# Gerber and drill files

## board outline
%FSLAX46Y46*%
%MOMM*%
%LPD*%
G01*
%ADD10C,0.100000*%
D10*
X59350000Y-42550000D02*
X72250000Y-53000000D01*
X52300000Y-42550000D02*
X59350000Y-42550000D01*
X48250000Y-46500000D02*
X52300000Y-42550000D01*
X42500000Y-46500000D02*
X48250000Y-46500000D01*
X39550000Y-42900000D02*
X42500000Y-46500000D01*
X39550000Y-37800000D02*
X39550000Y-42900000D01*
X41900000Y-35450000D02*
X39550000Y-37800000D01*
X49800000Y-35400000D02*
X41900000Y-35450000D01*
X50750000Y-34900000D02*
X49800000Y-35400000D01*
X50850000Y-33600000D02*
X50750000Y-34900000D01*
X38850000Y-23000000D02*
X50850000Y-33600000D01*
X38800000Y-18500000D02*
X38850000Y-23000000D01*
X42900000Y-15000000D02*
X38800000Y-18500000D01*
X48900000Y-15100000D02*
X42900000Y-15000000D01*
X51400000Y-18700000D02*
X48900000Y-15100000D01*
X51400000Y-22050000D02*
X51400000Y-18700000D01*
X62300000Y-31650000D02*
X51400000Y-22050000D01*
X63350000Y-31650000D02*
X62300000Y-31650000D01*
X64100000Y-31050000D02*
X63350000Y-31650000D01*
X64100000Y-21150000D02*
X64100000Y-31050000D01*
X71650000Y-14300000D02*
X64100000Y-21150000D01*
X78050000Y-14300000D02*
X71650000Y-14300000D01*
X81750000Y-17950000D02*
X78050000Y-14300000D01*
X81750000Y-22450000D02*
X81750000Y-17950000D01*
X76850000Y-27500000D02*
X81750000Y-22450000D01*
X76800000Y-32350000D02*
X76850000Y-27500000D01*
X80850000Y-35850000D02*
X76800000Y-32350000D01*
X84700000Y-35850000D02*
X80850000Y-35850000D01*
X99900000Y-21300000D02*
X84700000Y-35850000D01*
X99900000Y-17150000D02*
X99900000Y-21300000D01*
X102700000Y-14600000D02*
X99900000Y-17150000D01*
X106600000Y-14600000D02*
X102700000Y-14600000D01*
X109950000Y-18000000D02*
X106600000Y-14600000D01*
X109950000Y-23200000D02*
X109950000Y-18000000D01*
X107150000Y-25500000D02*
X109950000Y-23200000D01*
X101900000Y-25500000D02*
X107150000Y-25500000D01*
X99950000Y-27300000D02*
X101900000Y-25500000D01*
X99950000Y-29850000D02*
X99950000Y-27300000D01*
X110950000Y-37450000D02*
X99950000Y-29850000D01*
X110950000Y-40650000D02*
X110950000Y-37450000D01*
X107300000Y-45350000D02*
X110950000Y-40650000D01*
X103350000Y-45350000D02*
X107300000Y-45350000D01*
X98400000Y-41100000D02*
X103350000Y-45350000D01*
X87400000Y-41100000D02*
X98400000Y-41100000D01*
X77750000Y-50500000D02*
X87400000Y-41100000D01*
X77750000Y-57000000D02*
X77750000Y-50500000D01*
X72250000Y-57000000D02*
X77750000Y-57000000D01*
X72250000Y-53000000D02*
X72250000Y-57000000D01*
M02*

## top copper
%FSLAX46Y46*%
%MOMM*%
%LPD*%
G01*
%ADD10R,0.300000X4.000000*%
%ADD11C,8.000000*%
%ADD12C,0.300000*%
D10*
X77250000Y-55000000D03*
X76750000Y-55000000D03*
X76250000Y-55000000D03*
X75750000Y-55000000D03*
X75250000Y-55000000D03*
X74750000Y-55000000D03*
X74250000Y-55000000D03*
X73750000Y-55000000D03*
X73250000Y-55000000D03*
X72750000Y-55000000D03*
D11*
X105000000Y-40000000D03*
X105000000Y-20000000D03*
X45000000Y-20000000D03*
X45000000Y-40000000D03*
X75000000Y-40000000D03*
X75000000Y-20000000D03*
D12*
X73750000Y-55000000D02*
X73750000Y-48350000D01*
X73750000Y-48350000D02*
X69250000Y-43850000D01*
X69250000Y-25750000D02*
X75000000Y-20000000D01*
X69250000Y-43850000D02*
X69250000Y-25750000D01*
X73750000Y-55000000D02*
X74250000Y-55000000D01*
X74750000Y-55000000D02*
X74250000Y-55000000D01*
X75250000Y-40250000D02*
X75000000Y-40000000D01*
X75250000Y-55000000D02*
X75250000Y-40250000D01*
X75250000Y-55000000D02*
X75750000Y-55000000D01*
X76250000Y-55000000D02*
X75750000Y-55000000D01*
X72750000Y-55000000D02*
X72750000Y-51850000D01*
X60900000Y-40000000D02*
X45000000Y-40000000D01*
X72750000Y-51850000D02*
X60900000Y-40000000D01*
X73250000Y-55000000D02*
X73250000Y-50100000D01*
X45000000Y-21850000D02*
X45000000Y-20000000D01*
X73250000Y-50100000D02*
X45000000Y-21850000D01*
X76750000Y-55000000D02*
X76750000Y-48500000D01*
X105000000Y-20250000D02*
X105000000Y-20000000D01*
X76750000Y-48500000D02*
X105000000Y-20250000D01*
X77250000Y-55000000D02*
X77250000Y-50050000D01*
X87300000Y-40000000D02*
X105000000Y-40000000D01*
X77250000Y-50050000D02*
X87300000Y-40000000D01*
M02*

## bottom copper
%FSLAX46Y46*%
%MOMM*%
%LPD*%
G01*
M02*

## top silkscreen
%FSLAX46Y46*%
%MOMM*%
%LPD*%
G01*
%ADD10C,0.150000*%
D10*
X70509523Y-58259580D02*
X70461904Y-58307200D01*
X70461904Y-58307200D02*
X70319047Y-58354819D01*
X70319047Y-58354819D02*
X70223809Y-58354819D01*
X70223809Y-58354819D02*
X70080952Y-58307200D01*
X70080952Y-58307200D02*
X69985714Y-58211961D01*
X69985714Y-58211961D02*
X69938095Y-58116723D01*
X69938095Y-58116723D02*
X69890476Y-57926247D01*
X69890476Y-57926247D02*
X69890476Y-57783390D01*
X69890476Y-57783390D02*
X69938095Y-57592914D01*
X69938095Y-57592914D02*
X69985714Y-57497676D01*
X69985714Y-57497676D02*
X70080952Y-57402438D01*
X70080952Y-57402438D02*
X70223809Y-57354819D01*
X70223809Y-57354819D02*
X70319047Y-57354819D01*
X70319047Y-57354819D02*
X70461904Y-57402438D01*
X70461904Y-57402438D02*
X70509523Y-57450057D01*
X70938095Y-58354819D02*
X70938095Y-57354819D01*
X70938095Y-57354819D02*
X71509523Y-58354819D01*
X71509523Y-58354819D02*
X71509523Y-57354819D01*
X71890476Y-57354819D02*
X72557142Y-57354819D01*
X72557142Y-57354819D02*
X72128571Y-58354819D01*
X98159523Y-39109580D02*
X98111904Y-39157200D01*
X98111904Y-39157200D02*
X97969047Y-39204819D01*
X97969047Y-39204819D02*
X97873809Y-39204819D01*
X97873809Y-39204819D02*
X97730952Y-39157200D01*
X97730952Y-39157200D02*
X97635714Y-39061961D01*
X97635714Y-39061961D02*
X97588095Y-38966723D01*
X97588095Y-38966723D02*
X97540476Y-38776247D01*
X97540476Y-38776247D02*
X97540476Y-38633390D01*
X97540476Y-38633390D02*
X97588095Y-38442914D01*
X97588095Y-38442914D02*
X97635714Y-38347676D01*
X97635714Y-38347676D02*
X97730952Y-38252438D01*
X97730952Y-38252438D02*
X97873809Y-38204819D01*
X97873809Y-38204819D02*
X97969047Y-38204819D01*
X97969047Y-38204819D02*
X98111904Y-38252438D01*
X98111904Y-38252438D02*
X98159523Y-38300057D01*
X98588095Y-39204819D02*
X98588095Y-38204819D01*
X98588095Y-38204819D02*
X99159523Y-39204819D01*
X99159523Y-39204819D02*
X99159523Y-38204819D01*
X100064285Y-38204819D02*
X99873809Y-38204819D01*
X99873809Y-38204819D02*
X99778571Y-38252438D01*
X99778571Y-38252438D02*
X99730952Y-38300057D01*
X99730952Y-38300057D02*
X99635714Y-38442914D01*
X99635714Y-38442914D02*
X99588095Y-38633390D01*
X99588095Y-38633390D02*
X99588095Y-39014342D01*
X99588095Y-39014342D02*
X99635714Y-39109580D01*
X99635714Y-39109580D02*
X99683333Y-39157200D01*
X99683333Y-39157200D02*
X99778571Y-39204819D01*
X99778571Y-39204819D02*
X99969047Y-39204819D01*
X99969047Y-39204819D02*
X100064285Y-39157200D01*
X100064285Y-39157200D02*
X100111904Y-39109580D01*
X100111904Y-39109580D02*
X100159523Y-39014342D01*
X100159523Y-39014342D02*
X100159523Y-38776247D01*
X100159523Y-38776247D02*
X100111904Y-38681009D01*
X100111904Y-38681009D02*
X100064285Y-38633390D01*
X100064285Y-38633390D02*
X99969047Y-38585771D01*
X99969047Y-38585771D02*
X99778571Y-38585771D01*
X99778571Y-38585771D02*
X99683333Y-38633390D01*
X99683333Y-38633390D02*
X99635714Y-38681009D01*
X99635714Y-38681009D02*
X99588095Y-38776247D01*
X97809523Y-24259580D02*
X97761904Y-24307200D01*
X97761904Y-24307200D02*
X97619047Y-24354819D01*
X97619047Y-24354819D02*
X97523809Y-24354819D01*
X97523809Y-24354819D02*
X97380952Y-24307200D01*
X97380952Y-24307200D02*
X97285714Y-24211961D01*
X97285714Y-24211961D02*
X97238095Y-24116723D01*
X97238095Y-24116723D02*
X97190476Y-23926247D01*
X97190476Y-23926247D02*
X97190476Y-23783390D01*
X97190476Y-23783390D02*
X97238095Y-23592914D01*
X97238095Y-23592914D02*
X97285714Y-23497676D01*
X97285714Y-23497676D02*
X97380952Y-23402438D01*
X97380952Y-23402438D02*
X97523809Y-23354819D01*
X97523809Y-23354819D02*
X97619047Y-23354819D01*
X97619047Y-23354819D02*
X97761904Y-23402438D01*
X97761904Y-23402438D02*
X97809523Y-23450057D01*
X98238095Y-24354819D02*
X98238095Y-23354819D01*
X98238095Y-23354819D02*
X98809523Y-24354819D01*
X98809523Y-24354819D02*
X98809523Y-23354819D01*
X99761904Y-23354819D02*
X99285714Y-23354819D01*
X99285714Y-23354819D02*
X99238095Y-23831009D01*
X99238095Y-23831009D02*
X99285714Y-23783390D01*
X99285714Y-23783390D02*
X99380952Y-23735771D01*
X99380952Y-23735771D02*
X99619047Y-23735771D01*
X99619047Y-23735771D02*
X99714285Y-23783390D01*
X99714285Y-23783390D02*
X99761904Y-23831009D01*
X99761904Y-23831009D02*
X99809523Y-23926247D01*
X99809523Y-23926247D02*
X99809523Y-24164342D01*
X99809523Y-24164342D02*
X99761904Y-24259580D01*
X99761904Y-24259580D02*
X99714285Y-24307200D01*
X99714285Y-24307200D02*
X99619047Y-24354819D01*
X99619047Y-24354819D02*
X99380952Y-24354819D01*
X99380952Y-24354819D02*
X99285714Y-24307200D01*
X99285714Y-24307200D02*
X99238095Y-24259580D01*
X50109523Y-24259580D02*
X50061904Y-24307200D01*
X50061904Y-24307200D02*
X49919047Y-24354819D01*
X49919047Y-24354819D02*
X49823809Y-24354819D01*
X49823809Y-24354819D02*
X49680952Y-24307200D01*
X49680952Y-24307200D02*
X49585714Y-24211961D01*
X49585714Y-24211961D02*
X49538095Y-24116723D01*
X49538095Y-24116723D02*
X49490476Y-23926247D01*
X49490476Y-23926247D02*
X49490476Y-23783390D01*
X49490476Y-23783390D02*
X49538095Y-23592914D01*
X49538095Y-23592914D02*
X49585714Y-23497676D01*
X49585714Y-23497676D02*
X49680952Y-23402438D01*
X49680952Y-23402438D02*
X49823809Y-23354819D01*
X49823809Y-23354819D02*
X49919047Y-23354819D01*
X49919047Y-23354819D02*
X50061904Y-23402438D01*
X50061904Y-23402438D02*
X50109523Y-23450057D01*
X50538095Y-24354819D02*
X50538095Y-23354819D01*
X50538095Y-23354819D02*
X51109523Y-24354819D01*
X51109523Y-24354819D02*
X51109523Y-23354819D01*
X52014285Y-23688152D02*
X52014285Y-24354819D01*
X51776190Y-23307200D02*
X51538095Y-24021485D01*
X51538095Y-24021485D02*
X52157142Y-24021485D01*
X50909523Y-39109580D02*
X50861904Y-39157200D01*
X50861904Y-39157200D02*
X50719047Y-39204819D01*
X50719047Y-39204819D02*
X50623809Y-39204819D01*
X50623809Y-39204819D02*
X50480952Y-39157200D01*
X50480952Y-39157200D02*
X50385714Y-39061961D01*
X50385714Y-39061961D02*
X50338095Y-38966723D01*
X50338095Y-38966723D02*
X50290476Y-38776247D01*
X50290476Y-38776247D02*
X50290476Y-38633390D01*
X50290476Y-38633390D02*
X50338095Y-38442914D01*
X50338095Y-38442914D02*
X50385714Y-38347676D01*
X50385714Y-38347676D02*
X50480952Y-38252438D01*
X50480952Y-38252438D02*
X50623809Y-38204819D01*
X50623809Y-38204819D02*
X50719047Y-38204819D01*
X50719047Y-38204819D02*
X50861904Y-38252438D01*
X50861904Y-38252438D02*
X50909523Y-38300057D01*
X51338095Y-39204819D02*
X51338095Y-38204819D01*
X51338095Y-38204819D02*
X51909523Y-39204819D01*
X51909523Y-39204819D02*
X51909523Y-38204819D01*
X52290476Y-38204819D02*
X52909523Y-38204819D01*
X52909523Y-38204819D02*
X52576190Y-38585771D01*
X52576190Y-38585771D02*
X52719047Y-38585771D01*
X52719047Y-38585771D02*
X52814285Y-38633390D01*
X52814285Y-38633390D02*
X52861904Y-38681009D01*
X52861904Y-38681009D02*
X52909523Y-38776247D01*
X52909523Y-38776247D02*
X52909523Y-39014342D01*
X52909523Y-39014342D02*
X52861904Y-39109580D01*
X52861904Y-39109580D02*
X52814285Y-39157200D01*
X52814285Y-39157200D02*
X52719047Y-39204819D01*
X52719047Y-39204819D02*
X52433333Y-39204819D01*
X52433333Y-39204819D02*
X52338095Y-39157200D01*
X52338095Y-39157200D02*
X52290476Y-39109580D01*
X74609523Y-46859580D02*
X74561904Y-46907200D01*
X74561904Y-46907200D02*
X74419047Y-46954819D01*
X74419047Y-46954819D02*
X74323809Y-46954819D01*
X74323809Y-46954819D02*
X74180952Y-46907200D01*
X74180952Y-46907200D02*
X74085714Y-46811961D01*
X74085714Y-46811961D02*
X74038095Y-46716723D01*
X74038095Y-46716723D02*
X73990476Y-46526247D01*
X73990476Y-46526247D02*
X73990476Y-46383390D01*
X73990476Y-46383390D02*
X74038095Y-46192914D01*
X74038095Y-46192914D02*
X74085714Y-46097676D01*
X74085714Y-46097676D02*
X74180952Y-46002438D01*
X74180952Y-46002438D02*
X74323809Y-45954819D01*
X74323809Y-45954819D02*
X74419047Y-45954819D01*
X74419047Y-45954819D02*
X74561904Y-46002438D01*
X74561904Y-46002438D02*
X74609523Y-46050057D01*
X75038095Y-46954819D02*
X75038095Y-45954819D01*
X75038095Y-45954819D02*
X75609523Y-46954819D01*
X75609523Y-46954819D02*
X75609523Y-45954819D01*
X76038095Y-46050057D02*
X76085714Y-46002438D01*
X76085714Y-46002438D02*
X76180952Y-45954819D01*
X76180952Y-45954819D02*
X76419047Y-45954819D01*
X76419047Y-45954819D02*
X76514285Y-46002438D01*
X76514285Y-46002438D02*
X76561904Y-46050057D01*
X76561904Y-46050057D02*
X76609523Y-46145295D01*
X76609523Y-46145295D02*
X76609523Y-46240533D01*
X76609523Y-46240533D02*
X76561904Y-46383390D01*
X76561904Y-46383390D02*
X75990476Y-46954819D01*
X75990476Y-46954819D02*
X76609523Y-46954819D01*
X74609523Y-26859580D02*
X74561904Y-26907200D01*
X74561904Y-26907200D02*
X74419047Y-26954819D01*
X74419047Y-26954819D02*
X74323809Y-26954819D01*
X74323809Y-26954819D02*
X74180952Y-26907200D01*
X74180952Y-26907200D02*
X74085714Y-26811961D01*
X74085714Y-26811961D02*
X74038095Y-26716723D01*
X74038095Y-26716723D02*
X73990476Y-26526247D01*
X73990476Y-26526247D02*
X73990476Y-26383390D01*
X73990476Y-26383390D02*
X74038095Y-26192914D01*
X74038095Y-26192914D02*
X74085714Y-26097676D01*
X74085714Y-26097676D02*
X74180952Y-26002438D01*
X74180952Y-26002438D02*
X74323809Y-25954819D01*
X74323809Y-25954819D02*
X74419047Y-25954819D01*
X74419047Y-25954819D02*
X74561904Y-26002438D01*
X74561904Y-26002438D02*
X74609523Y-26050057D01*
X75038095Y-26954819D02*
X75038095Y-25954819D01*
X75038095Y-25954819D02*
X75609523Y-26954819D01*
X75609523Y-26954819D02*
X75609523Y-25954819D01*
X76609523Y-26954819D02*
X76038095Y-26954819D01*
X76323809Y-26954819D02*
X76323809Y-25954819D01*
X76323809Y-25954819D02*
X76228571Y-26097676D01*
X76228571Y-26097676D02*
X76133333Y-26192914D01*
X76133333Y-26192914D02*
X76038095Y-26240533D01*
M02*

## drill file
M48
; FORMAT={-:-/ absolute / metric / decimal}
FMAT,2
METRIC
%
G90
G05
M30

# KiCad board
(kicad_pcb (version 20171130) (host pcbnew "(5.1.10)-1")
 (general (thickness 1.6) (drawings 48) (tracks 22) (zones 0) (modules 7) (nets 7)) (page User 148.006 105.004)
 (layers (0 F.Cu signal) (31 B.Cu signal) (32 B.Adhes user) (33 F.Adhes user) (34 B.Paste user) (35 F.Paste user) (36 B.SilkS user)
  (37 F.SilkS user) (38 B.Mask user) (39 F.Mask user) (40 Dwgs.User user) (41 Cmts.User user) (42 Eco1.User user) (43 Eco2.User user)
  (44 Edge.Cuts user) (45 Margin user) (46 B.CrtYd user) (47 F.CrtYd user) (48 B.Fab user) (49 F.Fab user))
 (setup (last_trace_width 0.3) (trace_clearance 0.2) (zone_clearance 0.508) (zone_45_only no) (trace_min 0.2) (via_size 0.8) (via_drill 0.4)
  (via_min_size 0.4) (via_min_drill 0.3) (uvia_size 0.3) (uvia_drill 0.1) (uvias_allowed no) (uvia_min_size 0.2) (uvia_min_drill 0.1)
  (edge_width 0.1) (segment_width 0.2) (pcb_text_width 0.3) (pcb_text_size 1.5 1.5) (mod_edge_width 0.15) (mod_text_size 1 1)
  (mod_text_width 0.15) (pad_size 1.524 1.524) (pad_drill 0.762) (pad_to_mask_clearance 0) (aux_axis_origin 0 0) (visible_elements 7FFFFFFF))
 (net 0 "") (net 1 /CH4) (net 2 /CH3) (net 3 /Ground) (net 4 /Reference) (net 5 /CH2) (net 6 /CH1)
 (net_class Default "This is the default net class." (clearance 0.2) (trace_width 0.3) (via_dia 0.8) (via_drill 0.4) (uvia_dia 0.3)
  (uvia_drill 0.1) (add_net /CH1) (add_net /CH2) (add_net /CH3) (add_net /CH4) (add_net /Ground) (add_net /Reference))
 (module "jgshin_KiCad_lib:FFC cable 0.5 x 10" (layer F.Cu) (at 75 55)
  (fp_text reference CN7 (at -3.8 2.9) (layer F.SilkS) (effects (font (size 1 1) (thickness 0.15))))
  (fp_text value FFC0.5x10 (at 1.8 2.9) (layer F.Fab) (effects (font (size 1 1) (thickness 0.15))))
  (pad 10 smd rect (at 2.25 0) (size 0.3 4) (layers F.Cu F.Paste F.Mask) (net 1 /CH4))
  (pad 9 smd rect (at 1.75 0) (size 0.3 4) (layers F.Cu F.Paste F.Mask) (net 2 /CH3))
  (pad 8 smd rect (at 1.25 0) (size 0.3 4) (layers F.Cu F.Paste F.Mask) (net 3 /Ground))
  (pad 7 smd rect (at 0.75 0) (size 0.3 4) (layers F.Cu F.Paste F.Mask) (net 3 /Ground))
  (pad 6 smd rect (at 0.25 0) (size 0.3 4) (layers F.Cu F.Paste F.Mask) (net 3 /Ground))
  (pad 5 smd rect (at -0.25 0) (size 0.3 4) (layers F.Cu F.Paste F.Mask) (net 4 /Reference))
  (pad 4 smd rect (at -0.75 0) (size 0.3 4) (layers F.Cu F.Paste F.Mask) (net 4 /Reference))
  (pad 3 smd rect (at -1.25 0) (size 0.3 4) (layers F.Cu F.Paste F.Mask) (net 4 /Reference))
  (pad 2 smd rect (at -1.75 0) (size 0.3 4) (layers F.Cu F.Paste F.Mask) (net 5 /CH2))
  (pad 1 smd rect (at -2.25 0) (size 0.3 4) (layers F.Cu F.Paste F.Mask) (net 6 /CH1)))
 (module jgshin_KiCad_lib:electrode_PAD (layer F.Cu) (at 105 40)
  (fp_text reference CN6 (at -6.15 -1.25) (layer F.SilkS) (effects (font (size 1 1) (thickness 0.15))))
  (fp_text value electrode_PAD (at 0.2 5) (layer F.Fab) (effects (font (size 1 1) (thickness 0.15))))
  (pad 1 smd circle (at 0 0) (size 8 8) (layers F.Cu F.Paste F.Mask) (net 1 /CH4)))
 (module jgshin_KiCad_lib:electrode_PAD (layer F.Cu) (at 105 20)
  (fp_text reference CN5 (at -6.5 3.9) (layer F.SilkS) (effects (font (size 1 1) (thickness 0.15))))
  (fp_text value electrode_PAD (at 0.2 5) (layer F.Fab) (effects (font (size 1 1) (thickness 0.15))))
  (pad 1 smd circle (at 0 0) (size 8 8) (layers F.Cu F.Paste F.Mask) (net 2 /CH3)))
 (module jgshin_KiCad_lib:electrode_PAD (layer F.Cu) (at 45 20)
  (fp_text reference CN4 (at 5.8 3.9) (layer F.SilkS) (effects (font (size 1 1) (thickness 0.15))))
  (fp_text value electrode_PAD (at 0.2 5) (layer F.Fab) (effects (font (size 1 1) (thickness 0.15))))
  (pad 1 smd circle (at 0 0) (size 8 8) (layers F.Cu F.Paste F.Mask) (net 5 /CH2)))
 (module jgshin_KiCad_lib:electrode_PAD (layer F.Cu) (at 45 40)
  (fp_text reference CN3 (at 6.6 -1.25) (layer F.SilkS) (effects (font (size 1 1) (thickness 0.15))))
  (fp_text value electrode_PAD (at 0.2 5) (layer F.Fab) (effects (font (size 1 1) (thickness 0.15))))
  (pad 1 smd circle (at 0 0) (size 8 8) (layers F.Cu F.Paste F.Mask) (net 6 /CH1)))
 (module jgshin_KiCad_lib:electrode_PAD (layer F.Cu) (at 75 40)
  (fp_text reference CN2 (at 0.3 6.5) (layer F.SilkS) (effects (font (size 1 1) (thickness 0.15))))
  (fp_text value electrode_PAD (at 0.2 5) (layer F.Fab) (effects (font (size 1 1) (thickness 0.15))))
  (pad 1 smd circle (at 0 0) (size 8 8) (layers F.Cu F.Paste F.Mask) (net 3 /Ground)))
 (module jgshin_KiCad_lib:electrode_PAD (layer F.Cu) (at 75 20)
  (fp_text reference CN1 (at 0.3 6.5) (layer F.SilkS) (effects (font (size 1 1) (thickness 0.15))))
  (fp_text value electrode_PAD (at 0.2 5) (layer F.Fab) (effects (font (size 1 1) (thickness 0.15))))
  (pad 1 smd circle (at 0 0) (size 8 8) (layers F.Cu F.Paste F.Mask) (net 4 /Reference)))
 (gr_line (start 59.35 42.55) (end 72.25 53) (layer Edge.Cuts) (width 0.1))
 (gr_line (start 52.3 42.55) (end 59.35 42.55) (layer Edge.Cuts) (width 0.1))
 (gr_line (start 48.25 46.5) (end 52.3 42.55) (layer Edge.Cuts) (width 0.1))
 (gr_line (start 42.5 46.5) (end 48.25 46.5) (layer Edge.Cuts) (width 0.1))
 (gr_line (start 39.55 42.9) (end 42.5 46.5) (layer Edge.Cuts) (width 0.1))
 (gr_line (start 39.55 37.8) (end 39.55 42.9) (layer Edge.Cuts) (width 0.1))
 (gr_line (start 41.9 35.45) (end 39.55 37.8) (layer Edge.Cuts) (width 0.1))
 (gr_line (start 49.8 35.4) (end 41.9 35.45) (layer Edge.Cuts) (width 0.1))
 (gr_line (start 50.75 34.9) (end 49.8 35.4) (layer Edge.Cuts) (width 0.1))
 (gr_line (start 50.85 33.6) (end 50.75 34.9) (layer Edge.Cuts) (width 0.1))
 (gr_line (start 38.85 23) (end 50.85 33.6) (layer Edge.Cuts) (width 0.1))
 (gr_line (start 38.8 18.5) (end 38.85 23) (layer Edge.Cuts) (width 0.1))
 (gr_line (start 42.9 15) (end 38.8 18.5) (layer Edge.Cuts) (width 0.1))
 (gr_line (start 48.9 15.1) (end 42.9 15) (layer Edge.Cuts) (width 0.1))
 (gr_line (start 51.4 18.7) (end 48.9 15.1) (layer Edge.Cuts) (width 0.1))
 (gr_line (start 51.4 22.05) (end 51.4 18.7) (layer Edge.Cuts) (width 0.1))
 (gr_line (start 62.3 31.65) (end 51.4 22.05) (layer Edge.Cuts) (width 0.1))
 (gr_line (start 63.35 31.65) (end 62.3 31.65) (layer Edge.Cuts) (width 0.1))
 (gr_line (start 64.1 31.05) (end 63.35 31.65) (layer Edge.Cuts) (width 0.1))
 (gr_line (start 64.1 21.15) (end 64.1 31.05) (layer Edge.Cuts) (width 0.1))
 (gr_line (start 71.65 14.3) (end 64.1 21.15) (layer Edge.Cuts) (width 0.1))
 (gr_line (start 78.05 14.3) (end 71.65 14.3) (layer Edge.Cuts) (width 0.1))
 (gr_line (start 81.75 17.95) (end 78.05 14.3) (layer Edge.Cuts) (width 0.1))
 (gr_line (start 81.75 22.45) (end 81.75 17.95) (layer Edge.Cuts) (width 0.1))
 (gr_line (start 76.85 27.5) (end 81.75 22.45) (layer Edge.Cuts) (width 0.1))
 (gr_line (start 76.8 32.35) (end 76.85 27.5) (layer Edge.Cuts) (width 0.1))
 (gr_line (start 80.85 35.85) (end 76.8 32.35) (layer Edge.Cuts) (width 0.1))
 (gr_line (start 84.7 35.85) (end 80.85 35.85) (layer Edge.Cuts) (width 0.1))
 (gr_line (start 99.9 21.3) (end 84.7 35.85) (layer Edge.Cuts) (width 0.1))
 (gr_line (start 99.9 17.15) (end 99.9 21.3) (layer Edge.Cuts) (width 0.1))
 (gr_line (start 102.7 14.6) (end 99.9 17.15) (layer Edge.Cuts) (width 0.1))
 (gr_line (start 106.6 14.6) (end 102.7 14.6) (layer Edge.Cuts) (width 0.1))
 (gr_line (start 109.95 18) (end 106.6 14.6) (layer Edge.Cuts) (width 0.1))
 (gr_line (start 109.95 23.2) (end 109.95 18) (layer Edge.Cuts) (width 0.1))
 (gr_line (start 107.15 25.5) (end 109.95 23.2) (layer Edge.Cuts) (width 0.1))
 (gr_line (start 101.9 25.5) (end 107.15 25.5) (layer Edge.Cuts) (width 0.1))
 (gr_line (start 99.95 27.3) (end 101.9 25.5) (layer Edge.Cuts) (width 0.1))
 (gr_line (start 99.95 29.85) (end 99.95 27.3) (layer Edge.Cuts) (width 0.1))
 (gr_line (start 110.95 37.45) (end 99.95 29.85) (layer Edge.Cuts) (width 0.1))
 (gr_line (start 110.95 40.65) (end 110.95 37.45) (layer Edge.Cuts) (width 0.1))
 (gr_line (start 107.3 45.35) (end 110.95 40.65) (layer Edge.Cuts) (width 0.1))
 (gr_line (start 103.35 45.35) (end 107.3 45.35) (layer Edge.Cuts) (width 0.1))
 (gr_line (start 98.4 41.1) (end 103.35 45.35) (layer Edge.Cuts) (width 0.1))
 (gr_line (start 87.4 41.1) (end 98.4 41.1) (layer Edge.Cuts) (width 0.1))
 (gr_line (start 77.75 50.5) (end 87.4 41.1) (layer Edge.Cuts) (width 0.1))
 (gr_line (start 77.75 57) (end 77.75 50.5) (layer Edge.Cuts) (width 0.1))
 (gr_line (start 72.25 57) (end 77.75 57) (layer Edge.Cuts) (width 0.1))
 (gr_line (start 72.25 53) (end 72.25 57) (layer Edge.Cuts) (width 0.1))
 (segment (start 73.75 55) (end 73.75 48.35) (width 0.3) (layer F.Cu) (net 4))
 (segment (start 73.75 48.35) (end 69.25 43.85) (width 0.3) (layer F.Cu) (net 4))
 (segment (start 69.25 25.75) (end 75 20) (width 0.3) (layer F.Cu) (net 4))
 (segment (start 69.25 43.85) (end 69.25 25.75) (width 0.3) (layer F.Cu) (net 4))
 (segment (start 73.75 55) (end 74.25 55) (width 0.3) (layer F.Cu) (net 4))
 (segment (start 74.75 55) (end 74.25 55) (width 0.3) (layer F.Cu) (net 4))
 (segment (start 75.25 40.25) (end 75 40) (width 0.3) (layer F.Cu) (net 3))
 (segment (start 75.25 55) (end 75.25 40.25) (width 0.3) (layer F.Cu) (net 3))
 (segment (start 75.25 55) (end 75.75 55) (width 0.3) (layer F.Cu) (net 3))
 (segment (start 76.25 55) (end 75.75 55) (width 0.3) (layer F.Cu) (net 3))
 (segment (start 72.75 55) (end 72.75 51.85) (width 0.3) (layer F.Cu) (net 6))
 (segment (start 60.9 40) (end 45 40) (width 0.3) (layer F.Cu) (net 6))
 (segment (start 72.75 51.85) (end 60.9 40) (width 0.3) (layer F.Cu) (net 6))
 (segment (start 73.25 55) (end 73.25 50.1) (width 0.3) (layer F.Cu) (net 5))
 (segment (start 45 21.85) (end 45 20) (width 0.3) (layer F.Cu) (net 5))
 (segment (start 73.25 50.1) (end 45 21.85) (width 0.3) (layer F.Cu) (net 5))
 (segment (start 76.75 55) (end 76.75 48.5) (width 0.3) (layer F.Cu) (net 2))
 (segment (start 105 20.25) (end 105 20) (width 0.3) (layer F.Cu) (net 2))
 (segment (start 76.75 48.5) (end 105 20.25) (width 0.3) (layer F.Cu) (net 2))
 (segment (start 77.25 55) (end 77.25 50.05) (width 0.3) (layer F.Cu) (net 1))
 (segment (start 87.3 40) (end 105 40) (width 0.3) (layer F.Cu) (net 1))
 (segment (start 77.25 50.05) (end 87.3 40) (width 0.3) (layer F.Cu) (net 1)))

